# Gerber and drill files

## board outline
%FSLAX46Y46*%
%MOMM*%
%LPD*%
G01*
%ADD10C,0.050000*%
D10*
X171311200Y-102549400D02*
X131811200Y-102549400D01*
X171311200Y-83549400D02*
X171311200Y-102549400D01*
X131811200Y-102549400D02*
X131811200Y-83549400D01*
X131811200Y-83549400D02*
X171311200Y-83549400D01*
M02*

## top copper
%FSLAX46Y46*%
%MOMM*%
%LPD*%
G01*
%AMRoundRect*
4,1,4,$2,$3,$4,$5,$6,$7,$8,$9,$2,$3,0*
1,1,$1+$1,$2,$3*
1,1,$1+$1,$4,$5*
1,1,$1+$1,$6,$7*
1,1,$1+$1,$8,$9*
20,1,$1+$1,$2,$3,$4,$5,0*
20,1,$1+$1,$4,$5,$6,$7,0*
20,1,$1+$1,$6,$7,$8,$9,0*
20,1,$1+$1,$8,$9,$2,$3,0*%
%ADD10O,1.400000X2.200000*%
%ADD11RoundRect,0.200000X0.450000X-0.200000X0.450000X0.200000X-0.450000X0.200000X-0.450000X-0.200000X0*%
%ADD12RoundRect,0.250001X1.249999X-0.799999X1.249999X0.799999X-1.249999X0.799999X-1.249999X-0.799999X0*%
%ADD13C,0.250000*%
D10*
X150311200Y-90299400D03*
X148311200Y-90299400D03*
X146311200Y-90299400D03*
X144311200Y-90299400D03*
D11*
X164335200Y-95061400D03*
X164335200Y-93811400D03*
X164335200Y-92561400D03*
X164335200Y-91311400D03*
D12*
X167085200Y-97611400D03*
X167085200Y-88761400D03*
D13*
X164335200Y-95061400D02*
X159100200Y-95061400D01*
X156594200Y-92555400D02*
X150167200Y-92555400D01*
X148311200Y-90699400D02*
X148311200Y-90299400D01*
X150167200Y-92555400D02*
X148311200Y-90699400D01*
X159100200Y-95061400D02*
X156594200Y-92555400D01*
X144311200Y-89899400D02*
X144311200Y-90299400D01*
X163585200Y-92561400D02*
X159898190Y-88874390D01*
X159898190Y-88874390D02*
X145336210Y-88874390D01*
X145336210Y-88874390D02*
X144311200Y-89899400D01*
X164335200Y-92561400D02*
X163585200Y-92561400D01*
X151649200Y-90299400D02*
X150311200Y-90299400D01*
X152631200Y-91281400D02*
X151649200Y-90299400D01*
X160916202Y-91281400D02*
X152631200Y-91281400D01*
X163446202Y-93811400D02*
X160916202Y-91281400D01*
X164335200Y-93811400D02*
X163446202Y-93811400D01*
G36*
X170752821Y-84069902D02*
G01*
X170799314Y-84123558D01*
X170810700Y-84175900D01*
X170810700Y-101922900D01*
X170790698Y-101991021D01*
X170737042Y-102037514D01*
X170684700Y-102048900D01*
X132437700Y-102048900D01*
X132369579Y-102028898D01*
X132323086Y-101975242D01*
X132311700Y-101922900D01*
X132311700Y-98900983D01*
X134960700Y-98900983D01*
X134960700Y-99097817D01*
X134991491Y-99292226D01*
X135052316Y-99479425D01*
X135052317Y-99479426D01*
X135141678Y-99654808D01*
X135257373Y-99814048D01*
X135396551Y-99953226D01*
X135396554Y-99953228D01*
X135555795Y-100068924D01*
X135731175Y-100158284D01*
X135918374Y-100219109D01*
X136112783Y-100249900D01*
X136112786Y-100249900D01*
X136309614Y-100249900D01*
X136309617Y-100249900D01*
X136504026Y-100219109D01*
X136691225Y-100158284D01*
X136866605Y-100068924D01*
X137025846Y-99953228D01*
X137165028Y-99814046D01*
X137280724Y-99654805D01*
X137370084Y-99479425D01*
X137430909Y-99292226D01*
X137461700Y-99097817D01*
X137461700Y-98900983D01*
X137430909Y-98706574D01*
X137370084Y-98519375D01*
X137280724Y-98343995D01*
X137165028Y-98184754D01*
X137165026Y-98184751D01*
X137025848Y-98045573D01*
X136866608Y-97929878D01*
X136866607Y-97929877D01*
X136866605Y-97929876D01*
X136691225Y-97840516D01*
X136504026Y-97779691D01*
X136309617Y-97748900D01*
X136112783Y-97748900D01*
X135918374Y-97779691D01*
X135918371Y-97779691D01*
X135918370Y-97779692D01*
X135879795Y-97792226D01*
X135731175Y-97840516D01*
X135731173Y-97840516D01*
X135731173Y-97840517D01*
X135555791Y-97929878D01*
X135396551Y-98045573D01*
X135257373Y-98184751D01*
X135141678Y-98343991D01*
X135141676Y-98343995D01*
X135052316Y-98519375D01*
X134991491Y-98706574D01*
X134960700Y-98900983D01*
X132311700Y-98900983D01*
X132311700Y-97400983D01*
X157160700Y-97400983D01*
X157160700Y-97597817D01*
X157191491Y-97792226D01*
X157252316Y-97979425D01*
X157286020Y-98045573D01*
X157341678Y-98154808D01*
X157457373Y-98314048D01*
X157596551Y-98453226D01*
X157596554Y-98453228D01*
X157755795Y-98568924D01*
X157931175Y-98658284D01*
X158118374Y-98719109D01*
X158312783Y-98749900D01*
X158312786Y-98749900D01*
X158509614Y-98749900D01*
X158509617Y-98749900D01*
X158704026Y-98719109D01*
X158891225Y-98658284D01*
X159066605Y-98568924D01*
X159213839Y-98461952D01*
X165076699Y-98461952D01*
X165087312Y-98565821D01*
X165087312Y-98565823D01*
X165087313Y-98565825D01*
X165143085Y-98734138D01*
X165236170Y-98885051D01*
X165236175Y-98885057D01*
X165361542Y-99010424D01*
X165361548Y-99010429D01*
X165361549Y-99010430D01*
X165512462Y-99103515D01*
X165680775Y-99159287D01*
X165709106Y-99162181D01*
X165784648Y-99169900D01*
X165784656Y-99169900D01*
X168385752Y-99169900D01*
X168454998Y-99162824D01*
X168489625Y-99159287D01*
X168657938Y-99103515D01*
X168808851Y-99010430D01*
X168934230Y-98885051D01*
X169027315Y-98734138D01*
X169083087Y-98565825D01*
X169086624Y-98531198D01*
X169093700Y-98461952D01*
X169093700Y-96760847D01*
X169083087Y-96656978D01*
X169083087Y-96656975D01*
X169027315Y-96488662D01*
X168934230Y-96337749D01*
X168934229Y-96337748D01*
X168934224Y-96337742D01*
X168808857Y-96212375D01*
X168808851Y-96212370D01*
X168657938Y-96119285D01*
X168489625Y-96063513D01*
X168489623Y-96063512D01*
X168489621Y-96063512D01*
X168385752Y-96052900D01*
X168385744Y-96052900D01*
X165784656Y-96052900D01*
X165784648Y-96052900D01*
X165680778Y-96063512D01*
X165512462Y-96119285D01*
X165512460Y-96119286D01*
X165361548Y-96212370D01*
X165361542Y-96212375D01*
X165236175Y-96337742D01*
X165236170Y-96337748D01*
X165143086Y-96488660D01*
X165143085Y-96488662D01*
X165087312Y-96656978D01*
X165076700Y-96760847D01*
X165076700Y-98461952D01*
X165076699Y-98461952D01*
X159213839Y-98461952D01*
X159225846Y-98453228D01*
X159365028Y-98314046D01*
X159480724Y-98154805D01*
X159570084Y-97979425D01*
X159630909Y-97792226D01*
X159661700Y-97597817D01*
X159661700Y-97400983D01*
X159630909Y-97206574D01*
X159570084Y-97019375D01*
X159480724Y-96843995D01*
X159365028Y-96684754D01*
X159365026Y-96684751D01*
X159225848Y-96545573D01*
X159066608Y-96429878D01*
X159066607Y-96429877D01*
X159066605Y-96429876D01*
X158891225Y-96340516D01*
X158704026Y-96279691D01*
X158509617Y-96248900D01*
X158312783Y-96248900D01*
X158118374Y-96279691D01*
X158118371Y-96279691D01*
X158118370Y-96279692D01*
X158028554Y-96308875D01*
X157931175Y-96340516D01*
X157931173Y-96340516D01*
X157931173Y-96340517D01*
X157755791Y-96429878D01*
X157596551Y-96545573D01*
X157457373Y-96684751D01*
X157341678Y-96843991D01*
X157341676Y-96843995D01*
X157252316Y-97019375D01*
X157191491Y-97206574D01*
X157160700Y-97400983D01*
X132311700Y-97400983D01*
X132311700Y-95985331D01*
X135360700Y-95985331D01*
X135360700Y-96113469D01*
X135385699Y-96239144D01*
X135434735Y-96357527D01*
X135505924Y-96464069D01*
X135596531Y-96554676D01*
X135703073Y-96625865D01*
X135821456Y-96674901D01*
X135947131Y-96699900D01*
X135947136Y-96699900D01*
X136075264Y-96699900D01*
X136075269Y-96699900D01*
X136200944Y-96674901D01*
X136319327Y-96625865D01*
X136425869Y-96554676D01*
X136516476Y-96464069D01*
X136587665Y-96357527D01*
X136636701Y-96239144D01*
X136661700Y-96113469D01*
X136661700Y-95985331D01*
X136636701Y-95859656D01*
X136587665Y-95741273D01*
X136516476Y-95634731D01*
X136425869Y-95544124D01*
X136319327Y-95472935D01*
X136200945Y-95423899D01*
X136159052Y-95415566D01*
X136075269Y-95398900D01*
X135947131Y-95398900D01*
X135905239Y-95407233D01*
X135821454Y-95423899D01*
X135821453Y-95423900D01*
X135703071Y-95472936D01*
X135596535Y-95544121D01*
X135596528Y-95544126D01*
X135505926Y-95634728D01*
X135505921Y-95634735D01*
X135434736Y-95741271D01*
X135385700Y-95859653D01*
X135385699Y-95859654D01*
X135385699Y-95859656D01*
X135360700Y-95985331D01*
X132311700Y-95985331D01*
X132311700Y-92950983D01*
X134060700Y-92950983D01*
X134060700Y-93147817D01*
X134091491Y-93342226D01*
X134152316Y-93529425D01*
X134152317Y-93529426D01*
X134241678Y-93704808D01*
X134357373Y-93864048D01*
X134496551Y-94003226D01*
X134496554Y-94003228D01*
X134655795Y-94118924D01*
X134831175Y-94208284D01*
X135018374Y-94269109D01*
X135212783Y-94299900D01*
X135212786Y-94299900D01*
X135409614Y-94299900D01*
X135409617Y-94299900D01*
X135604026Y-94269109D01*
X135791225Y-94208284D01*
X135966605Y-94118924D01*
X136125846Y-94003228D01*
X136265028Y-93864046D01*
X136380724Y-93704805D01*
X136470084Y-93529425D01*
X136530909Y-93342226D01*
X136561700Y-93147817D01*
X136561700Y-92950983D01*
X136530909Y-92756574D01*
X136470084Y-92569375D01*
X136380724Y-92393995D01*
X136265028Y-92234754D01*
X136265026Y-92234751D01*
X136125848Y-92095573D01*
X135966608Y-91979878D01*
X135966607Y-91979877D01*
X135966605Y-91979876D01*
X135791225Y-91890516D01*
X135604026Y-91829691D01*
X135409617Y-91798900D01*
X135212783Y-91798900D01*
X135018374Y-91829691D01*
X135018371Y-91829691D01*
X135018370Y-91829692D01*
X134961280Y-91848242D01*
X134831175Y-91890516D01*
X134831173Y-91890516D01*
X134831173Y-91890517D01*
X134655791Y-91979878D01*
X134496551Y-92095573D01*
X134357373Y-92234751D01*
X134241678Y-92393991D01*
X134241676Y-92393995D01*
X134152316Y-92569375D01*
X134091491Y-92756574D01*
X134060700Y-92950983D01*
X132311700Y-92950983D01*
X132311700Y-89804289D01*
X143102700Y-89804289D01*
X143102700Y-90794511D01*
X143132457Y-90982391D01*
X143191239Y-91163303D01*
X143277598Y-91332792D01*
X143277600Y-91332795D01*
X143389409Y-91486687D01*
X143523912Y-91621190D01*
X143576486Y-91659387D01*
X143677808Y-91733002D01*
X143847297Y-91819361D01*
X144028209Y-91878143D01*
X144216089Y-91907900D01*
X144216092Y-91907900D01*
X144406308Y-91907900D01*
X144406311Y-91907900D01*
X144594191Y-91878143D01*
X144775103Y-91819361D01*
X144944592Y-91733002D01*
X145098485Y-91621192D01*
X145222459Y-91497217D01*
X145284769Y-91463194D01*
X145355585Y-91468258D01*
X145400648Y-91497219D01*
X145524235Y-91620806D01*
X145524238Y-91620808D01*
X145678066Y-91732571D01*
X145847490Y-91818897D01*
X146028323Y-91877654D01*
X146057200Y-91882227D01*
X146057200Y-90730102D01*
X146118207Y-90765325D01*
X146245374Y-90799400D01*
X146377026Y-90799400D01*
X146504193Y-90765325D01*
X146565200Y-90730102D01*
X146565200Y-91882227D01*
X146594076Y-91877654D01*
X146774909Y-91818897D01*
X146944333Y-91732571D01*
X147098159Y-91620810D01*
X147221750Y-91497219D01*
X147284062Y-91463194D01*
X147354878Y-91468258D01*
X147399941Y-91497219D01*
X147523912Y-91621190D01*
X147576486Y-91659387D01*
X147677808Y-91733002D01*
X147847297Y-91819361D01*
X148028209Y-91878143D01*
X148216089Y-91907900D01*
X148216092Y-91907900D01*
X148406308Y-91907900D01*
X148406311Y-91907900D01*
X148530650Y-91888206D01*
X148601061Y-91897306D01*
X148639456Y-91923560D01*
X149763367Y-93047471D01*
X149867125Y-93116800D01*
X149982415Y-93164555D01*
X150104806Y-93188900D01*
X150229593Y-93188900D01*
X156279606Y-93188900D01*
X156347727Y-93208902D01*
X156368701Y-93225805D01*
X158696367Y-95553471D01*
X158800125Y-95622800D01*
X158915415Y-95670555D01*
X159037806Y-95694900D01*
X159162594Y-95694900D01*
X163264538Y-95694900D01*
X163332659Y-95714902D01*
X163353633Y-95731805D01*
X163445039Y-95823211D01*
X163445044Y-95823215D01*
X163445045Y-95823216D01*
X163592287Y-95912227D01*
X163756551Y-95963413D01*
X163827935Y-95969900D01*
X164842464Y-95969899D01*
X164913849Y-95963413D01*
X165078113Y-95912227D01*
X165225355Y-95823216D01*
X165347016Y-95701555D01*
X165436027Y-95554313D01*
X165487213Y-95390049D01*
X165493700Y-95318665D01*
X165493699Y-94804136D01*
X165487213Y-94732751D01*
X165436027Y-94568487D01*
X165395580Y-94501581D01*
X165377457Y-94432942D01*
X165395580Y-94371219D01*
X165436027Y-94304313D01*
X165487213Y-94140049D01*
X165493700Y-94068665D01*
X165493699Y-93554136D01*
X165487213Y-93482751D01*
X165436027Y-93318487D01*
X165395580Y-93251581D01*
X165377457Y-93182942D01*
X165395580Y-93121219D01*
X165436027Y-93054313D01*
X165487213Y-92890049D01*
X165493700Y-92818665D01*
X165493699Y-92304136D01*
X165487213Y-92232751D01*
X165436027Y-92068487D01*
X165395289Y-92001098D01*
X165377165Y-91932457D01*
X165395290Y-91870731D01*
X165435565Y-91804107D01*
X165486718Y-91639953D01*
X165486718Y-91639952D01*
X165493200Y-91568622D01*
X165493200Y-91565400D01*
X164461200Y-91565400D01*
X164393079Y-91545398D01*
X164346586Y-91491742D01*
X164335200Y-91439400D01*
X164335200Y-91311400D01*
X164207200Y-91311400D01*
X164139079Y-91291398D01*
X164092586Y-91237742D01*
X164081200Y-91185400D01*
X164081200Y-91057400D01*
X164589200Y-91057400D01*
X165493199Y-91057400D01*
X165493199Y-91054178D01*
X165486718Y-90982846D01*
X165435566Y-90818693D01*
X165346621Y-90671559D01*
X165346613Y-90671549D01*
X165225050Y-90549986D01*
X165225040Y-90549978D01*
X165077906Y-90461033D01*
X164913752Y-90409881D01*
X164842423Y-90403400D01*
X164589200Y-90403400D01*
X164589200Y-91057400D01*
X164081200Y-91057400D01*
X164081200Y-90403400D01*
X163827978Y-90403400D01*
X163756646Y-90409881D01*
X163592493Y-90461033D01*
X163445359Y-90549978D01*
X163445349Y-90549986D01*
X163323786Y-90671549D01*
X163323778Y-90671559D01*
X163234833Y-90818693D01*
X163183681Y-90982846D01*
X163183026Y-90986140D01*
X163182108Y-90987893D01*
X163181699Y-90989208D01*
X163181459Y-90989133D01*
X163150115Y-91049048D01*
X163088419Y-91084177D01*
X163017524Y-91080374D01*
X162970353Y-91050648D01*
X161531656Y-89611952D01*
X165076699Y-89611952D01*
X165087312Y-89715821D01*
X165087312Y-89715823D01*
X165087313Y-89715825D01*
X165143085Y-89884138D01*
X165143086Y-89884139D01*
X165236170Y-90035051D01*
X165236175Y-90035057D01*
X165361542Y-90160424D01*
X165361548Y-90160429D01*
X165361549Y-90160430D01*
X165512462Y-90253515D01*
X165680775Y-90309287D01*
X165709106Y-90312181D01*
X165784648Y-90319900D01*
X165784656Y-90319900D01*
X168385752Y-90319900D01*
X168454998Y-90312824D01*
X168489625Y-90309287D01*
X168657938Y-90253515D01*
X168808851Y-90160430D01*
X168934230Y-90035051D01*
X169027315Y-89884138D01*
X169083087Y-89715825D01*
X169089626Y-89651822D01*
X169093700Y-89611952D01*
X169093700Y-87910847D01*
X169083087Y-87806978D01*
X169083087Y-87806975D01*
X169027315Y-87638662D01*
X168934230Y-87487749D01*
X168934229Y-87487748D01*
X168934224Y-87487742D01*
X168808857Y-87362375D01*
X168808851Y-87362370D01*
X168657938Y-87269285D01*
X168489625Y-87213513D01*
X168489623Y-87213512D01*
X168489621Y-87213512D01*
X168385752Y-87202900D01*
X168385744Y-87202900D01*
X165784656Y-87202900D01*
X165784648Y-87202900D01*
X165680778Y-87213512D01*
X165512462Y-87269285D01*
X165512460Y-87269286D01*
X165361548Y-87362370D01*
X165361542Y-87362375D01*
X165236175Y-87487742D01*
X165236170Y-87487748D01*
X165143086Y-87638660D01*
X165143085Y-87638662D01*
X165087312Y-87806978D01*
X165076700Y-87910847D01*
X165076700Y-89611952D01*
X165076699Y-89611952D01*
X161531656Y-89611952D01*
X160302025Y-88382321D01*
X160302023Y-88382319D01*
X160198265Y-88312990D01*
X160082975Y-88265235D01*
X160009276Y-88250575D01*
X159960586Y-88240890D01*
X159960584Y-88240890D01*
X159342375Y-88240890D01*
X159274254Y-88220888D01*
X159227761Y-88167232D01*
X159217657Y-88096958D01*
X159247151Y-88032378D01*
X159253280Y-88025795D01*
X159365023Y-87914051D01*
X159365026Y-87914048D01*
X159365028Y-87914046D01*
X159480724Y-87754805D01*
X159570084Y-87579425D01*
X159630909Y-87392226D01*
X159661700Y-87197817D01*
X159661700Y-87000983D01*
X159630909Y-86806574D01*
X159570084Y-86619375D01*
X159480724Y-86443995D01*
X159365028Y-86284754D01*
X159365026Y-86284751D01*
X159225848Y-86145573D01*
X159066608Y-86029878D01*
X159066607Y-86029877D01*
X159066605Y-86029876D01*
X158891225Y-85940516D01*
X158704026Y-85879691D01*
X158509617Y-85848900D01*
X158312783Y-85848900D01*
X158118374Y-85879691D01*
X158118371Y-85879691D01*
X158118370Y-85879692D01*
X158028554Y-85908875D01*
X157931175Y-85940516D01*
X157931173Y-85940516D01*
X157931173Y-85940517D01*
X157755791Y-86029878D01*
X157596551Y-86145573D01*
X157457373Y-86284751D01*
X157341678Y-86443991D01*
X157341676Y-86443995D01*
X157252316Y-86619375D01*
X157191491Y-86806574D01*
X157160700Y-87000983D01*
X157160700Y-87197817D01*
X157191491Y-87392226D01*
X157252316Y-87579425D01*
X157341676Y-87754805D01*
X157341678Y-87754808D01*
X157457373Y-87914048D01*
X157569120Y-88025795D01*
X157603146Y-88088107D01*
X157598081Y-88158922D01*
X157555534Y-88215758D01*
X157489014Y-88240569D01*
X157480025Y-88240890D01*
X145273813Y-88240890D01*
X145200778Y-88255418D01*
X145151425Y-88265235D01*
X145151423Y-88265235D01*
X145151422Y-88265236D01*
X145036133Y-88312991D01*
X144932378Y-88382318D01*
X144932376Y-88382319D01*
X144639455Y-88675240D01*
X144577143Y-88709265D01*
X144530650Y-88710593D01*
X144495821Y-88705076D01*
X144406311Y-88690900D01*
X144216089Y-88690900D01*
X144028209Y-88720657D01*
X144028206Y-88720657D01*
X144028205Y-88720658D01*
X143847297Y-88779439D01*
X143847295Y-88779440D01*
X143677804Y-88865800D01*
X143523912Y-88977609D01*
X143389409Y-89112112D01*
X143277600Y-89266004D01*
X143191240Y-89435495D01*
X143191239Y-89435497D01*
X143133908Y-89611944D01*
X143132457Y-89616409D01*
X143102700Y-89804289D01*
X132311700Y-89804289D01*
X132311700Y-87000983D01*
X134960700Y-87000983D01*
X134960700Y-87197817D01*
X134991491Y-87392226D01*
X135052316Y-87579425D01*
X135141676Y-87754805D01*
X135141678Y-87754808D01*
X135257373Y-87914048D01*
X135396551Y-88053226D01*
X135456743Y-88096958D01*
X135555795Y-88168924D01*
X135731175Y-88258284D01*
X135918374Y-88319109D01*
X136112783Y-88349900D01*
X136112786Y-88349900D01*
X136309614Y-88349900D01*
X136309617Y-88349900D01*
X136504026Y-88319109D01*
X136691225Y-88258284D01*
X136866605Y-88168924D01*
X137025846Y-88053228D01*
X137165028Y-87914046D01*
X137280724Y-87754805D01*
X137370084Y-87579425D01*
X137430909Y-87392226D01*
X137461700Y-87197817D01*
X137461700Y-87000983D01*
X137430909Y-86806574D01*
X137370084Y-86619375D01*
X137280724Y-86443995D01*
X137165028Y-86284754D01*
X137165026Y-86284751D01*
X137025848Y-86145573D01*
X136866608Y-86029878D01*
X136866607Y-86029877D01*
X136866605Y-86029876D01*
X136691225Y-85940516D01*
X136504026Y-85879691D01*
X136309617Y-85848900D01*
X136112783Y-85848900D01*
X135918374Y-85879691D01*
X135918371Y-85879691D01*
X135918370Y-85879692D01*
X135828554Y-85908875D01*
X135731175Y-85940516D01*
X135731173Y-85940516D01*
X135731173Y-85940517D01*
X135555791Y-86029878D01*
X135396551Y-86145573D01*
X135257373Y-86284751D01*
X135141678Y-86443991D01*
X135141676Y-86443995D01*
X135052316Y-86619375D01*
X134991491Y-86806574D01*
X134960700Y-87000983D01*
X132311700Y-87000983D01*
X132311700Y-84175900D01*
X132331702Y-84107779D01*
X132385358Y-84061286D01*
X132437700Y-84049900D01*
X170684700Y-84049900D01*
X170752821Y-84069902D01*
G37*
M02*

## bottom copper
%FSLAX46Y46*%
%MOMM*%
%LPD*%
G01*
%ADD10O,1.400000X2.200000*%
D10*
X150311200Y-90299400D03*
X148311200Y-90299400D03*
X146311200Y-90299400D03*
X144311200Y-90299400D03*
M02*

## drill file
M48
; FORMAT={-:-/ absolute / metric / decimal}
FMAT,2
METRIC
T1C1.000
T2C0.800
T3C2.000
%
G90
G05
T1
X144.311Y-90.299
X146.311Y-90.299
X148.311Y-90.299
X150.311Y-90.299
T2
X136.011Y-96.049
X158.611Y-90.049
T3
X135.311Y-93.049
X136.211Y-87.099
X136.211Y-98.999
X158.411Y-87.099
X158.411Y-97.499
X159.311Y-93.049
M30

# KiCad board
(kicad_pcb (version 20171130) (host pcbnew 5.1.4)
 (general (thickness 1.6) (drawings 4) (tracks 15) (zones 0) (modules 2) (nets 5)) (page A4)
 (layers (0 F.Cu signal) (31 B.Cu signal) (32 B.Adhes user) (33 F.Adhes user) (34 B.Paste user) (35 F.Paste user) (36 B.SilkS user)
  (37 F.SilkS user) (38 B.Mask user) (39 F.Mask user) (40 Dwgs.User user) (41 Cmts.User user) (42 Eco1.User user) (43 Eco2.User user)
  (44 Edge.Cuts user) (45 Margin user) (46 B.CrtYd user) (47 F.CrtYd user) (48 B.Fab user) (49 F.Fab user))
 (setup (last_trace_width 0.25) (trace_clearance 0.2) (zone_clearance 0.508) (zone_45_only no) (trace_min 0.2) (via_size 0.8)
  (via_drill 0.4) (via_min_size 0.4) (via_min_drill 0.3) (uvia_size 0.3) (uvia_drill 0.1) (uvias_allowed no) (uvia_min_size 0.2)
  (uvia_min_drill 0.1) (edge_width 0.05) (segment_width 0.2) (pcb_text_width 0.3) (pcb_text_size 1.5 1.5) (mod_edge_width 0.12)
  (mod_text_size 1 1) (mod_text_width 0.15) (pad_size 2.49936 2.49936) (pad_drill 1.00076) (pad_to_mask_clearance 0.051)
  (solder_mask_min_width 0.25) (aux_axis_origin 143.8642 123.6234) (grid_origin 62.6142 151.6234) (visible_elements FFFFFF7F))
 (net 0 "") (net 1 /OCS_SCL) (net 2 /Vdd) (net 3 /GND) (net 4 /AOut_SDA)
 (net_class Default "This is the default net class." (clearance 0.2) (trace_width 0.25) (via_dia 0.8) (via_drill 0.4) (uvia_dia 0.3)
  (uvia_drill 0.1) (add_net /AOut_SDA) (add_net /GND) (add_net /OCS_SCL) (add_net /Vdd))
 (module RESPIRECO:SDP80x (layer F.Cu) (at 147.3112 93.0494 180)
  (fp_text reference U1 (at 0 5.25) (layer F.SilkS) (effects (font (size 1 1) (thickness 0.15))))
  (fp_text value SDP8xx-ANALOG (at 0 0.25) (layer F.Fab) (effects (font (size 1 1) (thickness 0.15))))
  (pad 1 thru_hole oval (at -3 2.75 180) (size 1.4 2.2) (drill 1) (layers *.Cu *.Mask) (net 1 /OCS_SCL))
  (pad 2 thru_hole oval (at -1 2.75 180) (size 1.4 2.2) (drill 1) (layers *.Cu *.Mask) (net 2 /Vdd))
  (pad 3 thru_hole oval (at 1 2.75 180) (size 1.4 2.2) (drill 1) (layers *.Cu *.Mask) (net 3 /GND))
  (pad 4 thru_hole oval (at 3 2.75 180) (size 1.4 2.2) (drill 1) (layers *.Cu *.Mask) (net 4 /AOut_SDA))
  (pad "" np_thru_hole circle (at -11.1 5.95 180) (size 2 2) (drill 2) (layers *.Cu *.Mask))
  (pad "" np_thru_hole circle (at -11.1 -4.45 180) (size 2 2) (drill 2) (layers *.Cu *.Mask))
  (pad "" np_thru_hole circle (at 11.1 -5.95 180) (size 2 2) (drill 2) (layers *.Cu *.Mask))
  (pad "" np_thru_hole circle (at 11.1 5.95 180) (size 2 2) (drill 2) (layers *.Cu *.Mask))
  (pad "" np_thru_hole circle (at -11.3 3 180) (size 0.8 0.8) (drill 0.8) (layers *.Cu *.Mask))
  (pad "" np_thru_hole circle (at -12 0 180) (size 2 2) (drill 2) (layers *.Cu *.Mask))
  (pad "" np_thru_hole circle (at 11.3 -3 180) (size 0.8 0.8) (drill 0.8) (layers *.Cu *.Mask))
  (pad "" np_thru_hole circle (at 12 0 180) (size 2 2) (drill 2) (layers *.Cu *.Mask)))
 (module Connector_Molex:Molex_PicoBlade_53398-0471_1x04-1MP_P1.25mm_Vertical (layer F.Cu) (at 165.5852 93.1864 90)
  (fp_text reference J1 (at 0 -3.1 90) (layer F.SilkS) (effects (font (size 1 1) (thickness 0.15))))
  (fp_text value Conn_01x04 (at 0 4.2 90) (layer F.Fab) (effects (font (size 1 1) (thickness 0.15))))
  (pad 1 smd roundrect (at -1.875 -1.25 90) (size 0.8 1.3) (layers F.Cu F.Paste F.Mask) (roundrect_rratio 0.25) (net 2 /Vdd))
  (pad 2 smd roundrect (at -0.625 -1.25 90) (size 0.8 1.3) (layers F.Cu F.Paste F.Mask) (roundrect_rratio 0.25) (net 1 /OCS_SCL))
  (pad 3 smd roundrect (at 0.625 -1.25 90) (size 0.8 1.3) (layers F.Cu F.Paste F.Mask) (roundrect_rratio 0.25) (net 4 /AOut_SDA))
  (pad 4 smd roundrect (at 1.875 -1.25 90) (size 0.8 1.3) (layers F.Cu F.Paste F.Mask) (roundrect_rratio 0.25) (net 3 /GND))
  (pad MP smd roundrect (at -4.425 1.5 90) (size 2.1 3) (layers F.Cu F.Paste F.Mask) (roundrect_rratio 0.119048))
  (pad MP smd roundrect (at 4.425 1.5 90) (size 2.1 3) (layers F.Cu F.Paste F.Mask) (roundrect_rratio 0.119048)))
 (gr_line (start 171.3112 102.5494) (end 131.8112 102.5494) (layer Edge.Cuts) (width 0.05))
 (gr_line (start 171.3112 83.5494) (end 171.3112 102.5494) (layer Edge.Cuts) (width 0.05))
 (gr_line (start 131.8112 102.5494) (end 131.8112 83.5494) (layer Edge.Cuts) (width 0.05))
 (gr_line (start 131.8112 83.5494) (end 171.3112 83.5494) (layer Edge.Cuts) (width 0.05))
 (segment (start 164.3352 95.0614) (end 159.1002 95.0614) (width 0.25) (layer F.Cu) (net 2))
 (segment (start 156.5942 92.5554) (end 150.1672 92.5554) (width 0.25) (layer F.Cu) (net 2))
 (segment (start 148.3112 90.6994) (end 148.3112 90.2994) (width 0.25) (layer F.Cu) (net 2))
 (segment (start 150.1672 92.5554) (end 148.3112 90.6994) (width 0.25) (layer F.Cu) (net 2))
 (segment (start 159.1002 95.0614) (end 156.5942 92.5554) (width 0.25) (layer F.Cu) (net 2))
 (segment (start 144.3112 89.8994) (end 144.3112 90.2994) (width 0.25) (layer F.Cu) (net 4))
 (segment (start 163.5852 92.5614) (end 159.89819 88.87439) (width 0.25) (layer F.Cu) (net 4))
 (segment (start 159.89819 88.87439) (end 145.33621 88.87439) (width 0.25) (layer F.Cu) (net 4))
 (segment (start 145.33621 88.87439) (end 144.3112 89.8994) (width 0.25) (layer F.Cu) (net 4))
 (segment (start 164.3352 92.5614) (end 163.5852 92.5614) (width 0.25) (layer F.Cu) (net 4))
 (segment (start 151.6492 90.2994) (end 150.3112 90.2994) (width 0.25) (layer F.Cu) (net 1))
 (segment (start 152.6312 91.2814) (end 151.6492 90.2994) (width 0.25) (layer F.Cu) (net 1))
 (segment (start 160.916202 91.2814) (end 152.6312 91.2814) (width 0.25) (layer F.Cu) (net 1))
 (segment (start 163.446202 93.8114) (end 160.916202 91.2814) (width 0.25) (layer F.Cu) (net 1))
 (segment (start 164.3352 93.8114) (end 163.446202 93.8114) (width 0.25) (layer F.Cu) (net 1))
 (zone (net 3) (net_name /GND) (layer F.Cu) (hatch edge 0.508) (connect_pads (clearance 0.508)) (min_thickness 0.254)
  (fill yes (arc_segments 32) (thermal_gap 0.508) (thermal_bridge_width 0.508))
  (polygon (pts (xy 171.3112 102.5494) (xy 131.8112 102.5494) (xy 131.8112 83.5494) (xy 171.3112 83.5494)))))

